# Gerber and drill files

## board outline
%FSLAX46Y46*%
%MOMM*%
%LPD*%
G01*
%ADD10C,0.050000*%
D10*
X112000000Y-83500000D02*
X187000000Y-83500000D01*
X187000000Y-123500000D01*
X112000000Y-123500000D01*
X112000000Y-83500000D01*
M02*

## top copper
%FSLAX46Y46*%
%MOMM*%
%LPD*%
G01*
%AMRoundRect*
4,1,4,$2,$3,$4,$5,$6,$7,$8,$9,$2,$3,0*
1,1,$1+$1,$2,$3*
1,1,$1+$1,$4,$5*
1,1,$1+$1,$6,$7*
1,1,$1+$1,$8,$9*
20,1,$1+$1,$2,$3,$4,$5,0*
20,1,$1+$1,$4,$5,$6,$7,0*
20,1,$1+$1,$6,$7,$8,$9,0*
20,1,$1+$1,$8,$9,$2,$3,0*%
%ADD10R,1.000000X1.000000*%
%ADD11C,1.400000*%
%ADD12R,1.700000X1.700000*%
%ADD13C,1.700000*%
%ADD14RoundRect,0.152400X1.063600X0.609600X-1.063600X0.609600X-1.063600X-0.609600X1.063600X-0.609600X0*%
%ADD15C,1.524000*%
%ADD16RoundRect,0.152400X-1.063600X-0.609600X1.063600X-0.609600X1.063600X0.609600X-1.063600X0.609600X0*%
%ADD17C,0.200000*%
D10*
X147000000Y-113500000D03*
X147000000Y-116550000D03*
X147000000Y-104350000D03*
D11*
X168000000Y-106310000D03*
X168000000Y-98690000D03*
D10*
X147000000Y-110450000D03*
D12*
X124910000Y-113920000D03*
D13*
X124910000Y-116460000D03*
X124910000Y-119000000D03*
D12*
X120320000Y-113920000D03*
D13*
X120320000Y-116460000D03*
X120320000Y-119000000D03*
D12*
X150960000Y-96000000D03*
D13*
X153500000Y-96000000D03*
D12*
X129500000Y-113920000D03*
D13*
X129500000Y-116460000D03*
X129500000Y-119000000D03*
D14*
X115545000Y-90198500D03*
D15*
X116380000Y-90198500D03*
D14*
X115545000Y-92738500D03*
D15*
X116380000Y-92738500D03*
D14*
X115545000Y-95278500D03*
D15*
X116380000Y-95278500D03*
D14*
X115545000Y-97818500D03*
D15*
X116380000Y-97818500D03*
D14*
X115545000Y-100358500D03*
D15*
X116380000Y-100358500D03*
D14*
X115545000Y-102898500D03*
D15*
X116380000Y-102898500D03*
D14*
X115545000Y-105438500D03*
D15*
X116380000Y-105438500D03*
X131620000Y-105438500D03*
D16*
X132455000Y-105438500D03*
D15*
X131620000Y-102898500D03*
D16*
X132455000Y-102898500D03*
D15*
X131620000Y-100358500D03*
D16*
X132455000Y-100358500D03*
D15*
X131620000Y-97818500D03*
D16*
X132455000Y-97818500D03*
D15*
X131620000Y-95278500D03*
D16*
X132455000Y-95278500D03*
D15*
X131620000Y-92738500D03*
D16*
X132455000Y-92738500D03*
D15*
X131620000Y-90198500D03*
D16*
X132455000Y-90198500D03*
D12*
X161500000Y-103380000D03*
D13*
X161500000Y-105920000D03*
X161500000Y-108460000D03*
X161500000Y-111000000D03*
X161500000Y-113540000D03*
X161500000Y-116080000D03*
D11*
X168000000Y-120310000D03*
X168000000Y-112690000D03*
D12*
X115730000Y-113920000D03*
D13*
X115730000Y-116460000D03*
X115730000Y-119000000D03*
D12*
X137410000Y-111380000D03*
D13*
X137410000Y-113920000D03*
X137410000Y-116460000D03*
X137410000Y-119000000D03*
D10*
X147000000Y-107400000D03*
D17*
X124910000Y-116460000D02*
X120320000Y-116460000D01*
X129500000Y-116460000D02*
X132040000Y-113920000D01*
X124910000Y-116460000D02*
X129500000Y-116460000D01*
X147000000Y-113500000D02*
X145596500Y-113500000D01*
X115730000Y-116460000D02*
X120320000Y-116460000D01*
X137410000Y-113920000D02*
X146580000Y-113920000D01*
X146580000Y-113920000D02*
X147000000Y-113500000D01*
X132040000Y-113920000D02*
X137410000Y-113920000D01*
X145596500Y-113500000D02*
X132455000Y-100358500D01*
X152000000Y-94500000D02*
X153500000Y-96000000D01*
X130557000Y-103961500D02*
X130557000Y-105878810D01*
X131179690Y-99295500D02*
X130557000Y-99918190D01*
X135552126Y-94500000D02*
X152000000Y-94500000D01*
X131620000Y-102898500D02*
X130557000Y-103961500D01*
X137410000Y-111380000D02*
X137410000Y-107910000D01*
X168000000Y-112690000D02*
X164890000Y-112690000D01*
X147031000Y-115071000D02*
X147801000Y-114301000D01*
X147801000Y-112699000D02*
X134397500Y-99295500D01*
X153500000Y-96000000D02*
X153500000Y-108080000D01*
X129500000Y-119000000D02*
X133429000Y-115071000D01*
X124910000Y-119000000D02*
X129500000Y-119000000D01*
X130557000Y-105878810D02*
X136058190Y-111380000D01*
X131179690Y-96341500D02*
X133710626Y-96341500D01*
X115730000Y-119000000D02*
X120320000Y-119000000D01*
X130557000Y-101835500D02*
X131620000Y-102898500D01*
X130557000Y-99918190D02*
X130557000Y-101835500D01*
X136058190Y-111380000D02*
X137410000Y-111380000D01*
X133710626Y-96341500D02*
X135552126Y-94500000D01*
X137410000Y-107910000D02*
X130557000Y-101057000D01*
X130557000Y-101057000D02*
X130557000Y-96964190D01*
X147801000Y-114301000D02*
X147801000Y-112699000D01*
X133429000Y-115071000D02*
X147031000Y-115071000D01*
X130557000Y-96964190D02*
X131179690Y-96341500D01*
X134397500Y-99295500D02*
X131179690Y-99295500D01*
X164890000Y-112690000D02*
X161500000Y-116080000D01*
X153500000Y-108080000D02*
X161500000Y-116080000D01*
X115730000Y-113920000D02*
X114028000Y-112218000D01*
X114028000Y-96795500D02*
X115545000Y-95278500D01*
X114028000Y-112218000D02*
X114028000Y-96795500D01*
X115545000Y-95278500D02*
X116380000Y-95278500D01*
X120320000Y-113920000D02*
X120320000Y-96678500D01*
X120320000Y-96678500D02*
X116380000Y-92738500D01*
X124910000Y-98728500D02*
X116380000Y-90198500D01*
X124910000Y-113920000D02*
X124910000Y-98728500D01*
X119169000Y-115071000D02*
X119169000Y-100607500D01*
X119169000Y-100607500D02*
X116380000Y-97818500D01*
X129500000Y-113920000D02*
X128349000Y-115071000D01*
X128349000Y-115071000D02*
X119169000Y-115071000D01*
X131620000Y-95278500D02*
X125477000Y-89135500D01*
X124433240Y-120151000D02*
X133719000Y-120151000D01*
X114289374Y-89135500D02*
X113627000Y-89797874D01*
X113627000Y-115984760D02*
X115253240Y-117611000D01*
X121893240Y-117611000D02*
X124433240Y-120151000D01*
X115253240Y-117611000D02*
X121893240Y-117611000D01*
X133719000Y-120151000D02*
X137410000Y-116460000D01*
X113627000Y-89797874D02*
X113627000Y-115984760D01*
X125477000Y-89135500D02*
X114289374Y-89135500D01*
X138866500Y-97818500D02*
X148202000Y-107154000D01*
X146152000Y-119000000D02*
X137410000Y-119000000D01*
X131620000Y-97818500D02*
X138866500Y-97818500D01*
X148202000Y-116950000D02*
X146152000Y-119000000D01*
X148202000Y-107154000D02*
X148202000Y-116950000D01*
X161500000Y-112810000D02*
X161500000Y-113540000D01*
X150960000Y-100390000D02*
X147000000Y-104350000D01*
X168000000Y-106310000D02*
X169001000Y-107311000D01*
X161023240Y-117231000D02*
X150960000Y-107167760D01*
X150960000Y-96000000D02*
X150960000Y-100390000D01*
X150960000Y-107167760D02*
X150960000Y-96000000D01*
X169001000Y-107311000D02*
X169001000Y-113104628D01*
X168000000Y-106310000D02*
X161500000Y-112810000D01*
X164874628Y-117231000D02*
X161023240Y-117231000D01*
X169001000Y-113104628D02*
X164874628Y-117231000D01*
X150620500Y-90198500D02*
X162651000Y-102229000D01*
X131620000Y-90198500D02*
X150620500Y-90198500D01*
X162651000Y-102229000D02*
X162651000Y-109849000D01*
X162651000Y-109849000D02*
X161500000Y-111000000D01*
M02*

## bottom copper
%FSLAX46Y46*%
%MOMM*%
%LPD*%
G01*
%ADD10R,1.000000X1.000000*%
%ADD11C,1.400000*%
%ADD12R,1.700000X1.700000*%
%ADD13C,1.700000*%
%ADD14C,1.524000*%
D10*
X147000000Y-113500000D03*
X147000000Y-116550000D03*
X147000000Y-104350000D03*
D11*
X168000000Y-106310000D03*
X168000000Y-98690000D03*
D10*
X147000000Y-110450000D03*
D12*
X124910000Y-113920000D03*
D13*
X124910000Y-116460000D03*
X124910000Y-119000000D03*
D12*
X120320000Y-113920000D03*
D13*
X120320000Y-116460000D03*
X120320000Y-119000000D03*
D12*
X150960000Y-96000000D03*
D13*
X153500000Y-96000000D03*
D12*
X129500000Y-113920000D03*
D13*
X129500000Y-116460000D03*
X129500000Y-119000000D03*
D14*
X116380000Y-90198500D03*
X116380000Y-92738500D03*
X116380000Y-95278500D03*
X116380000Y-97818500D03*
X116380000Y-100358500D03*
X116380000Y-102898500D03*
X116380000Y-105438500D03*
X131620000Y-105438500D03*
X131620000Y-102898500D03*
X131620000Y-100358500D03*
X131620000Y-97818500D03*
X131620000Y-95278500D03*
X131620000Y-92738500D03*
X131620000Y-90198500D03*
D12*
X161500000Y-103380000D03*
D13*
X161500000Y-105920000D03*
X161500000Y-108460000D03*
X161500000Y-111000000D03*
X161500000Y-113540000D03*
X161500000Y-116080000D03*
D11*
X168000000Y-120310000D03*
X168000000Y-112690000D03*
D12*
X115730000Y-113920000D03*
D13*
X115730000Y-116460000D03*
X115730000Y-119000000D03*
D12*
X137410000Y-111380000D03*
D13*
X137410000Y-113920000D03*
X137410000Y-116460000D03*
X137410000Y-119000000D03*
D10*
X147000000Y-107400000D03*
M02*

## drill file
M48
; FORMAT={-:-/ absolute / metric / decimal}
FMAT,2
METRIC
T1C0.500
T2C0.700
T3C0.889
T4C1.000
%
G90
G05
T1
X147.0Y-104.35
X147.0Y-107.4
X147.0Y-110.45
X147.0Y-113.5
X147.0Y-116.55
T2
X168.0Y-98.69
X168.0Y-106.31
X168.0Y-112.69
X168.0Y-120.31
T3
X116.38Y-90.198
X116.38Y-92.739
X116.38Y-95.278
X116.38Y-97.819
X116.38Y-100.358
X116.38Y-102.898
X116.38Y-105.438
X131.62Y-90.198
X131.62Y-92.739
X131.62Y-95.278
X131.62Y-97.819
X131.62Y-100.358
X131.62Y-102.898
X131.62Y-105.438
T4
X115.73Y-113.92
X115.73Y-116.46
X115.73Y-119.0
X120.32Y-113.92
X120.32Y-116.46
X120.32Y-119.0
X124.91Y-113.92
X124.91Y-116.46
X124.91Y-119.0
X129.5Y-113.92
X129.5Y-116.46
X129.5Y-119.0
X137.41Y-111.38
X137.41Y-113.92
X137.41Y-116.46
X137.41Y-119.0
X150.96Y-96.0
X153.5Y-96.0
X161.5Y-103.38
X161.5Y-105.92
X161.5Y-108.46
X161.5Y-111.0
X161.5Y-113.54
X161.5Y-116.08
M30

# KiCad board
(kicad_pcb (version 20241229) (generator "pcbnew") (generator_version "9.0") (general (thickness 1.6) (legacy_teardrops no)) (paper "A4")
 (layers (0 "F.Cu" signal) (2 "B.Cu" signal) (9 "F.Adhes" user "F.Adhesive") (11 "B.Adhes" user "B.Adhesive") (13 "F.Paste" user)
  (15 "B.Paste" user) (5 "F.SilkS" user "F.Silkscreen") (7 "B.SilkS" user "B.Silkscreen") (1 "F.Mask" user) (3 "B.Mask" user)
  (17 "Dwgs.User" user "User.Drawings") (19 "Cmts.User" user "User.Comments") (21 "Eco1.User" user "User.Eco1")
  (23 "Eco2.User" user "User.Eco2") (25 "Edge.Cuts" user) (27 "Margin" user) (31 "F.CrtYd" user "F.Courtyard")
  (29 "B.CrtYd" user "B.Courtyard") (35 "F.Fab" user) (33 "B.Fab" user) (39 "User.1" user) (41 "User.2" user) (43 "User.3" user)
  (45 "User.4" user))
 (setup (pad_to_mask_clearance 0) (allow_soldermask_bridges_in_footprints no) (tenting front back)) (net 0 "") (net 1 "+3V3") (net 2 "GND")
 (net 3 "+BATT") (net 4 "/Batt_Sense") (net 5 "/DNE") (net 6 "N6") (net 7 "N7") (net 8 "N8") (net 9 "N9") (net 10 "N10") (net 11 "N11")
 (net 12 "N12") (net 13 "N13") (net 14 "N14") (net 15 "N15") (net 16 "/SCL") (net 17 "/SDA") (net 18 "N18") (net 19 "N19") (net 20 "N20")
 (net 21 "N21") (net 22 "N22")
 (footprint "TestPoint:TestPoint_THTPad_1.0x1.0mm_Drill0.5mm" (layer "F.Cu") (at 147 113.5)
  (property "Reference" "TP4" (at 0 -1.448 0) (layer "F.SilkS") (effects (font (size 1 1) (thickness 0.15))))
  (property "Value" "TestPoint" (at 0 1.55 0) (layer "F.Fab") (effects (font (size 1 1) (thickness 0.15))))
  (pad "1" thru_hole rect (at 0 0) (size 1 1) (drill 0.5) (layers "*.Cu" "*.Mask") (remove_unused_layers no) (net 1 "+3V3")))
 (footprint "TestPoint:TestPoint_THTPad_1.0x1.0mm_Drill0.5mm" (layer "F.Cu") (at 147 116.55)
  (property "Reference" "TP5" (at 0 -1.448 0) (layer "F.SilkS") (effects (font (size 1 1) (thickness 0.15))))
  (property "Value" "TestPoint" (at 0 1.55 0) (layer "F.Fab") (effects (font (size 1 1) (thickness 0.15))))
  (pad "1" thru_hole rect (at 0 0) (size 1 1) (drill 0.5) (layers "*.Cu" "*.Mask") (remove_unused_layers no) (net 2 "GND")))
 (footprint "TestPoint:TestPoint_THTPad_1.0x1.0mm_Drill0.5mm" (layer "F.Cu") (at 147 104.35)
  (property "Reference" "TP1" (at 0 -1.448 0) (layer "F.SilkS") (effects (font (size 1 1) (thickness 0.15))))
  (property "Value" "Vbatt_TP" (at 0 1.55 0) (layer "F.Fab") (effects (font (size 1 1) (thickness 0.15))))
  (pad "1" thru_hole rect (at 0 0) (size 1 1) (drill 0.5) (layers "*.Cu" "*.Mask") (remove_unused_layers no) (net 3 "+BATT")))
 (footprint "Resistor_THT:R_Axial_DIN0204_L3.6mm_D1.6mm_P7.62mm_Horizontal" (layer "F.Cu") (at 168 106.31 90)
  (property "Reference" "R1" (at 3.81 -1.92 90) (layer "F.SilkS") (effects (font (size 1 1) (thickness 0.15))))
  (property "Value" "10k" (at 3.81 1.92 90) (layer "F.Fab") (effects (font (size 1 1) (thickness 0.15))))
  (pad "1" thru_hole circle (at 0 0 90) (size 1.4 1.4) (drill 0.7) (layers "*.Cu" "*.Mask") (remove_unused_layers no) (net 3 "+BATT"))
  (pad "2" thru_hole circle (at 7.62 0 90) (size 1.4 1.4) (drill 0.7) (layers "*.Cu" "*.Mask") (remove_unused_layers no)
   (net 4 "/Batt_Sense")))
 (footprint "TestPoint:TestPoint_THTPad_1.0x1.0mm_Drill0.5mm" (layer "F.Cu") (at 147 110.45)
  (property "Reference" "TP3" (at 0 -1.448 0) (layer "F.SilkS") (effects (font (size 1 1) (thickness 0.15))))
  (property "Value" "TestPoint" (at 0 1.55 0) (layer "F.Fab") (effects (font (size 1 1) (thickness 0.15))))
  (pad "1" thru_hole rect (at 0 0) (size 1 1) (drill 0.5) (layers "*.Cu" "*.Mask") (remove_unused_layers no) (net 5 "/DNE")))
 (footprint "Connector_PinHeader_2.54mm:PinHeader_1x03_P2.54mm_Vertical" (layer "F.Cu") (at 124.91 113.92)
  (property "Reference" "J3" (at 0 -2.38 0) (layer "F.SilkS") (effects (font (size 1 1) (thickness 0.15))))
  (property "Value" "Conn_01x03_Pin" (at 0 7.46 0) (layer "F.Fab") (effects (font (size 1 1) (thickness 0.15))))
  (pad "1" thru_hole rect (at 0 0) (size 1.7 1.7) (drill 1) (layers "*.Cu" "*.Mask") (remove_unused_layers no) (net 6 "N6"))
  (pad "2" thru_hole circle (at 0 2.54) (size 1.7 1.7) (drill 1) (layers "*.Cu" "*.Mask") (remove_unused_layers no) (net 1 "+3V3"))
  (pad "3" thru_hole circle (at 0 5.08) (size 1.7 1.7) (drill 1) (layers "*.Cu" "*.Mask") (remove_unused_layers no) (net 2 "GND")))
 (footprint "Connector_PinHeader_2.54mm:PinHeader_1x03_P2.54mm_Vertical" (layer "F.Cu") (at 120.32 113.92)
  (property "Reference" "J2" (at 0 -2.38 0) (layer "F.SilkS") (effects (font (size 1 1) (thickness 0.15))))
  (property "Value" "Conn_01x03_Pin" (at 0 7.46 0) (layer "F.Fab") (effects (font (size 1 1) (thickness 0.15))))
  (pad "1" thru_hole rect (at 0 0) (size 1.7 1.7) (drill 1) (layers "*.Cu" "*.Mask") (remove_unused_layers no) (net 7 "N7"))
  (pad "2" thru_hole circle (at 0 2.54) (size 1.7 1.7) (drill 1) (layers "*.Cu" "*.Mask") (remove_unused_layers no) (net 1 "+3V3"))
  (pad "3" thru_hole circle (at 0 5.08) (size 1.7 1.7) (drill 1) (layers "*.Cu" "*.Mask") (remove_unused_layers no) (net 2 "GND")))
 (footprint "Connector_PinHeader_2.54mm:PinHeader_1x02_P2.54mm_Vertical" (layer "F.Cu") (at 150.96 96 90)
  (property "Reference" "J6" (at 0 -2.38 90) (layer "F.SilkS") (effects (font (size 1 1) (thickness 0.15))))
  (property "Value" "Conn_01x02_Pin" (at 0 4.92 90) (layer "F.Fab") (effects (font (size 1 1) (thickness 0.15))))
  (pad "1" thru_hole rect (at 0 0 90) (size 1.7 1.7) (drill 1) (layers "*.Cu" "*.Mask") (remove_unused_layers no) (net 3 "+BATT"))
  (pad "2" thru_hole circle (at 0 2.54 90) (size 1.7 1.7) (drill 1) (layers "*.Cu" "*.Mask") (remove_unused_layers no) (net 2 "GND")))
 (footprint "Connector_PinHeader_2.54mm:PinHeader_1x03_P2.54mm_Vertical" (layer "F.Cu") (at 129.5 113.92)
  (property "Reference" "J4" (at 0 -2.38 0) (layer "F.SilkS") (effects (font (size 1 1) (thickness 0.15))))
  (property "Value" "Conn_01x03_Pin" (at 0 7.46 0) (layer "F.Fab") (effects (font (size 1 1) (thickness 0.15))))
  (pad "1" thru_hole rect (at 0 0) (size 1.7 1.7) (drill 1) (layers "*.Cu" "*.Mask") (remove_unused_layers no) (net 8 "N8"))
  (pad "2" thru_hole circle (at 0 2.54) (size 1.7 1.7) (drill 1) (layers "*.Cu" "*.Mask") (remove_unused_layers no) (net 1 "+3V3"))
  (pad "3" thru_hole circle (at 0 5.08) (size 1.7 1.7) (drill 1) (layers "*.Cu" "*.Mask") (remove_unused_layers no) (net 2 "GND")))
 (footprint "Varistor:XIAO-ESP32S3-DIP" (layer "F.Cu") (at 124 97.8185)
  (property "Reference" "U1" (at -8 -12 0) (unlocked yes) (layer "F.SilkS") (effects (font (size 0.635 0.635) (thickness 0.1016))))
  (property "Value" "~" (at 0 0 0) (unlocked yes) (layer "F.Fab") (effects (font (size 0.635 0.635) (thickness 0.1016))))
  (pad "1" smd roundrect (at -8.455 -7.62 180) (size 2.432 1.524) (layers "F.Cu" "F.Mask") (roundrect_rratio 0.1) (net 6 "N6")
   (thermal_bridge_angle 45))
  (pad "1" thru_hole circle (at -7.62 -7.62 180) (size 1.524 1.524) (drill 0.889) (layers "*.Cu" "*.Mask") (remove_unused_layers no)
   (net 6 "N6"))
  (pad "2" smd roundrect (at -8.455 -5.08 180) (size 2.432 1.524) (layers "F.Cu" "F.Mask") (roundrect_rratio 0.1) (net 7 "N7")
   (thermal_bridge_angle 45))
  (pad "2" thru_hole circle (at -7.62 -5.08 180) (size 1.524 1.524) (drill 0.889) (layers "*.Cu" "*.Mask") (remove_unused_layers no)
   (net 7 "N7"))
  (pad "3" smd roundrect (at -8.455 -2.54 180) (size 2.432 1.524) (layers "F.Cu" "F.Mask") (roundrect_rratio 0.1) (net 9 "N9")
   (thermal_bridge_angle 45))
  (pad "3" thru_hole circle (at -7.62 -2.54 180) (size 1.524 1.524) (drill 0.889) (layers "*.Cu" "*.Mask") (remove_unused_layers no)
   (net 9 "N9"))
  (pad "4" smd roundrect (at -8.455 0 180) (size 2.432 1.524) (layers "F.Cu" "F.Mask") (roundrect_rratio 0.1) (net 8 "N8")
   (thermal_bridge_angle 45))
  (pad "4" thru_hole circle (at -7.62 0 180) (size 1.524 1.524) (drill 0.889) (layers "*.Cu" "*.Mask") (remove_unused_layers no)
   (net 8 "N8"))
  (pad "5" smd roundrect (at -8.455 2.54 180) (size 2.432 1.524) (layers "F.Cu" "F.Mask") (roundrect_rratio 0.1) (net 4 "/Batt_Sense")
   (thermal_bridge_angle 45))
  (pad "5" thru_hole circle (at -7.62 2.54 180) (size 1.524 1.524) (drill 0.889) (layers "*.Cu" "*.Mask") (remove_unused_layers no)
   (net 4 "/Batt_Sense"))
  (pad "6" smd roundrect (at -8.455 5.08 180) (size 2.432 1.524) (layers "F.Cu" "F.Mask") (roundrect_rratio 0.1) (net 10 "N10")
   (thermal_bridge_angle 45))
  (pad "6" thru_hole circle (at -7.62 5.08 180) (size 1.524 1.524) (drill 0.889) (layers "*.Cu" "*.Mask") (remove_unused_layers no)
   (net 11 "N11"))
  (pad "7" smd roundrect (at -8.455 7.62 180) (size 2.432 1.524) (layers "F.Cu" "F.Mask") (roundrect_rratio 0.1) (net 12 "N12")
   (thermal_bridge_angle 45))
  (pad "7" thru_hole circle (at -7.62 7.62 180) (size 1.524 1.524) (drill 0.889) (layers "*.Cu" "*.Mask") (remove_unused_layers no)
   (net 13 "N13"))
  (pad "8" thru_hole circle (at 7.62 7.62) (size 1.524 1.524) (drill 0.889) (layers "*.Cu" "*.Mask") (remove_unused_layers no)
   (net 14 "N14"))
  (pad "8" smd roundrect (at 8.455 7.62) (size 2.432 1.524) (layers "F.Cu" "F.Mask") (roundrect_rratio 0.1) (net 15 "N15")
   (thermal_bridge_angle 45))
  (pad "9" thru_hole circle (at 7.62 5.08) (size 1.524 1.524) (drill 0.889) (layers "*.Cu" "*.Mask") (remove_unused_layers no) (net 2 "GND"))
  (pad "9" smd roundrect (at 8.455 5.08) (size 2.432 1.524) (layers "F.Cu" "F.Mask") (roundrect_rratio 0.1) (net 2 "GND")
   (thermal_bridge_angle 45))
  (pad "10" thru_hole circle (at 7.62 2.54) (size 1.524 1.524) (drill 0.889) (layers "*.Cu" "*.Mask") (remove_unused_layers no)
   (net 1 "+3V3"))
  (pad "10" smd roundrect (at 8.455 2.54) (size 2.432 1.524) (layers "F.Cu" "F.Mask") (roundrect_rratio 0.1) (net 1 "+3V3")
   (thermal_bridge_angle 45))
  (pad "11" thru_hole circle (at 7.62 0) (size 1.524 1.524) (drill 0.889) (layers "*.Cu" "*.Mask") (remove_unused_layers no) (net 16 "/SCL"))
  (pad "11" smd roundrect (at 8.455 0) (size 2.432 1.524) (layers "F.Cu" "F.Mask") (roundrect_rratio 0.1) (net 16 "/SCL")
   (thermal_bridge_angle 45))
  (pad "12" thru_hole circle (at 7.62 -2.54) (size 1.524 1.524) (drill 0.889) (layers "*.Cu" "*.Mask") (remove_unused_layers no)
   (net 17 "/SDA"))
  (pad "12" smd roundrect (at 8.455 -2.54) (size 2.432 1.524) (layers "F.Cu" "F.Mask") (roundrect_rratio 0.1) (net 17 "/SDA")
   (thermal_bridge_angle 45))
  (pad "13" thru_hole circle (at 7.62 -5.08) (size 1.524 1.524) (drill 0.889) (layers "*.Cu" "*.Mask") (remove_unused_layers no)
   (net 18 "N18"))
  (pad "13" smd roundrect (at 8.455 -5.08) (size 2.432 1.524) (layers "F.Cu" "F.Mask") (roundrect_rratio 0.1) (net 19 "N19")
   (thermal_bridge_angle 45))
  (pad "14" thru_hole circle (at 7.62 -7.62) (size 1.524 1.524) (drill 0.889) (layers "*.Cu" "*.Mask") (remove_unused_layers no)
   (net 5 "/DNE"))
  (pad "14" smd roundrect (at 8.455 -7.62) (size 2.432 1.524) (layers "F.Cu" "F.Mask") (roundrect_rratio 0.1) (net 5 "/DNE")
   (thermal_bridge_angle 45)))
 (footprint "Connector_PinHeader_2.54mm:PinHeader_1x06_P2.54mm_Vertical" (layer "F.Cu") (at 161.5 103.38)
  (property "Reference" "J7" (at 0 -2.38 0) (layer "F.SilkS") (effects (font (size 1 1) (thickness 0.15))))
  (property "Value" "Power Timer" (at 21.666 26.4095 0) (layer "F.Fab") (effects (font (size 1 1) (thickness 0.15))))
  (pad "1" thru_hole rect (at 0 0) (size 1.7 1.7) (drill 1) (layers "*.Cu" "*.Mask") (remove_unused_layers no) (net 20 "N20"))
  (pad "2" thru_hole circle (at 0 2.54) (size 1.7 1.7) (drill 1) (layers "*.Cu" "*.Mask") (remove_unused_layers no) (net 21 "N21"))
  (pad "3" thru_hole circle (at 0 5.08) (size 1.7 1.7) (drill 1) (layers "*.Cu" "*.Mask") (remove_unused_layers no) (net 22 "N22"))
  (pad "4" thru_hole circle (at 0 7.62) (size 1.7 1.7) (drill 1) (layers "*.Cu" "*.Mask") (remove_unused_layers no) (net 5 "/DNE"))
  (pad "5" thru_hole circle (at 0 10.16) (size 1.7 1.7) (drill 1) (layers "*.Cu" "*.Mask") (remove_unused_layers no) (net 3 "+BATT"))
  (pad "6" thru_hole circle (at 0 12.7) (size 1.7 1.7) (drill 1) (layers "*.Cu" "*.Mask") (remove_unused_layers no) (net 2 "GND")))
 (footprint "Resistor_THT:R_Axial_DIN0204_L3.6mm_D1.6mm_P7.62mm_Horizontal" (layer "F.Cu") (at 168 120.31 90)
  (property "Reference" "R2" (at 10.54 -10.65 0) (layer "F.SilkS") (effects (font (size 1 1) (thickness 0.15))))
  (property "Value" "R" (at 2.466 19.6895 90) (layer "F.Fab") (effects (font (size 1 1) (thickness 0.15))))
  (pad "1" thru_hole circle (at 0 0 90) (size 1.4 1.4) (drill 0.7) (layers "*.Cu" "*.Mask") (remove_unused_layers no) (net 4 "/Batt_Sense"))
  (pad "2" thru_hole circle (at 7.62 0 90) (size 1.4 1.4) (drill 0.7) (layers "*.Cu" "*.Mask") (remove_unused_layers no) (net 2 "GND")))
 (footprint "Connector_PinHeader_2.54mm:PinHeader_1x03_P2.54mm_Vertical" (layer "F.Cu") (at 115.73 113.92)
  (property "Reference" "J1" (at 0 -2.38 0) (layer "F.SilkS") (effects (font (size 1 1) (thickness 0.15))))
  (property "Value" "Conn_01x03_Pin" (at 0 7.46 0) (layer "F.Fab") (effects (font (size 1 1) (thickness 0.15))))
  (pad "1" thru_hole rect (at 0 0) (size 1.7 1.7) (drill 1) (layers "*.Cu" "*.Mask") (remove_unused_layers no) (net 9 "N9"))
  (pad "2" thru_hole circle (at 0 2.54) (size 1.7 1.7) (drill 1) (layers "*.Cu" "*.Mask") (remove_unused_layers no) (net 1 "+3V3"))
  (pad "3" thru_hole circle (at 0 5.08) (size 1.7 1.7) (drill 1) (layers "*.Cu" "*.Mask") (remove_unused_layers no) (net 2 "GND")))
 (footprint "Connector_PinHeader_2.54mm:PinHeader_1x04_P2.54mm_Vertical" (layer "F.Cu") (at 137.41 111.38)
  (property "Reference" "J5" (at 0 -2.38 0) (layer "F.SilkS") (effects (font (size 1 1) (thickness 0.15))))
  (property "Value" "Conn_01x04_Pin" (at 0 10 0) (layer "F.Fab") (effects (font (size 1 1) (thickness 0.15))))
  (pad "1" thru_hole rect (at 0 0) (size 1.7 1.7) (drill 1) (layers "*.Cu" "*.Mask") (remove_unused_layers no) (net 2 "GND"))
  (pad "2" thru_hole circle (at 0 2.54) (size 1.7 1.7) (drill 1) (layers "*.Cu" "*.Mask") (remove_unused_layers no) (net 1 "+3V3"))
  (pad "3" thru_hole circle (at 0 5.08) (size 1.7 1.7) (drill 1) (layers "*.Cu" "*.Mask") (remove_unused_layers no) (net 17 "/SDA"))
  (pad "4" thru_hole circle (at 0 7.62) (size 1.7 1.7) (drill 1) (layers "*.Cu" "*.Mask") (remove_unused_layers no) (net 16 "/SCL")))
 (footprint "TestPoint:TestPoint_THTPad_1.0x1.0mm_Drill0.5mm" (layer "F.Cu") (at 147 107.4)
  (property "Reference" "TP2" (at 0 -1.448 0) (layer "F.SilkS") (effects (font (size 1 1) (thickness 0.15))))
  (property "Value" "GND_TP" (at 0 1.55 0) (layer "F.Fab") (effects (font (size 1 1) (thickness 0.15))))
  (pad "1" thru_hole rect (at 0 0) (size 1 1) (drill 0.5) (layers "*.Cu" "*.Mask") (remove_unused_layers no) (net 2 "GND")))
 (gr_rect (start 112 83.5) (end 187 123.5) (stroke (width 0.05) (type default)) (fill no) (layer "Edge.Cuts"))
 (segment (start 124.91 116.46) (end 120.32 116.46) (width 0.2) (layer "F.Cu") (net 1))
 (segment (start 129.5 116.46) (end 132.04 113.92) (width 0.2) (layer "F.Cu") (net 1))
 (segment (start 124.91 116.46) (end 129.5 116.46) (width 0.2) (layer "F.Cu") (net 1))
 (segment (start 147 113.5) (end 145.5965 113.5) (width 0.2) (layer "F.Cu") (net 1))
 (segment (start 115.73 116.46) (end 120.32 116.46) (width 0.2) (layer "F.Cu") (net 1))
 (segment (start 137.41 113.92) (end 146.58 113.92) (width 0.2) (layer "F.Cu") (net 1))
 (segment (start 146.58 113.92) (end 147 113.5) (width 0.2) (layer "F.Cu") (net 1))
 (segment (start 132.04 113.92) (end 137.41 113.92) (width 0.2) (layer "F.Cu") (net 1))
 (segment (start 145.5965 113.5) (end 132.455 100.3585) (width 0.2) (layer "F.Cu") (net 1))
 (segment (start 152 94.5) (end 153.5 96) (width 0.2) (layer "F.Cu") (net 2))
 (segment (start 130.557 103.9615) (end 130.557 105.87881) (width 0.2) (layer "F.Cu") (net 2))
 (segment (start 131.17969 99.2955) (end 130.557 99.91819) (width 0.2) (layer "F.Cu") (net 2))
 (segment (start 135.552126 94.5) (end 152 94.5) (width 0.2) (layer "F.Cu") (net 2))
 (segment (start 131.62 102.8985) (end 130.557 103.9615) (width 0.2) (layer "F.Cu") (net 2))
 (segment (start 137.41 111.38) (end 137.41 107.91) (width 0.2) (layer "F.Cu") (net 2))
 (segment (start 168 112.69) (end 164.89 112.69) (width 0.2) (layer "F.Cu") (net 2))
 (segment (start 147.031 115.071) (end 147.801 114.301) (width 0.2) (layer "F.Cu") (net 2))
 (segment (start 147.801 112.699) (end 134.3975 99.2955) (width 0.2) (layer "F.Cu") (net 2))
 (segment (start 153.5 96) (end 153.5 108.08) (width 0.2) (layer "F.Cu") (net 2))
 (segment (start 129.5 119) (end 133.429 115.071) (width 0.2) (layer "F.Cu") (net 2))
 (segment (start 124.91 119) (end 129.5 119) (width 0.2) (layer "F.Cu") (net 2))
 (segment (start 130.557 105.87881) (end 136.05819 111.38) (width 0.2) (layer "F.Cu") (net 2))
 (segment (start 131.17969 96.3415) (end 133.710626 96.3415) (width 0.2) (layer "F.Cu") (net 2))
 (segment (start 115.73 119) (end 120.32 119) (width 0.2) (layer "F.Cu") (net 2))
 (segment (start 130.557 101.8355) (end 131.62 102.8985) (width 0.2) (layer "F.Cu") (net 2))
 (segment (start 130.557 99.91819) (end 130.557 101.8355) (width 0.2) (layer "F.Cu") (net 2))
 (segment (start 136.05819 111.38) (end 137.41 111.38) (width 0.2) (layer "F.Cu") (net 2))
 (segment (start 133.710626 96.3415) (end 135.552126 94.5) (width 0.2) (layer "F.Cu") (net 2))
 (segment (start 137.41 107.91) (end 130.557 101.057) (width 0.2) (layer "F.Cu") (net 2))
 (segment (start 130.557 101.057) (end 130.557 96.96419) (width 0.2) (layer "F.Cu") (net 2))
 (segment (start 147.801 114.301) (end 147.801 112.699) (width 0.2) (layer "F.Cu") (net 2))
 (segment (start 133.429 115.071) (end 147.031 115.071) (width 0.2) (layer "F.Cu") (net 2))
 (segment (start 130.557 96.96419) (end 131.17969 96.3415) (width 0.2) (layer "F.Cu") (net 2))
 (segment (start 134.3975 99.2955) (end 131.17969 99.2955) (width 0.2) (layer "F.Cu") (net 2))
 (segment (start 164.89 112.69) (end 161.5 116.08) (width 0.2) (layer "F.Cu") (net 2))
 (segment (start 153.5 108.08) (end 161.5 116.08) (width 0.2) (layer "F.Cu") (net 2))
 (segment (start 115.73 113.92) (end 114.028 112.218) (width 0.2) (layer "F.Cu") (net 9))
 (segment (start 114.028 96.7955) (end 115.545 95.2785) (width 0.2) (layer "F.Cu") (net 9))
 (segment (start 114.028 112.218) (end 114.028 96.7955) (width 0.2) (layer "F.Cu") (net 9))
 (segment (start 115.545 95.2785) (end 116.38 95.2785) (width 0.2) (layer "F.Cu") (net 9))
 (segment (start 120.32 113.92) (end 120.32 96.6785) (width 0.2) (layer "F.Cu") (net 7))
 (segment (start 120.32 96.6785) (end 116.38 92.7385) (width 0.2) (layer "F.Cu") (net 7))
 (segment (start 124.91 98.7285) (end 116.38 90.1985) (width 0.2) (layer "F.Cu") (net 6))
 (segment (start 124.91 113.92) (end 124.91 98.7285) (width 0.2) (layer "F.Cu") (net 6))
 (segment (start 119.169 115.071) (end 119.169 100.6075) (width 0.2) (layer "F.Cu") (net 8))
 (segment (start 119.169 100.6075) (end 116.38 97.8185) (width 0.2) (layer "F.Cu") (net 8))
 (segment (start 129.5 113.92) (end 128.349 115.071) (width 0.2) (layer "F.Cu") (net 8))
 (segment (start 128.349 115.071) (end 119.169 115.071) (width 0.2) (layer "F.Cu") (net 8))
 (segment (start 131.62 95.2785) (end 125.477 89.1355) (width 0.2) (layer "F.Cu") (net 17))
 (segment (start 124.43324 120.151) (end 133.719 120.151) (width 0.2) (layer "F.Cu") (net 17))
 (segment (start 114.289374 89.1355) (end 113.627 89.797874) (width 0.2) (layer "F.Cu") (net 17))
 (segment (start 113.627 115.98476) (end 115.25324 117.611) (width 0.2) (layer "F.Cu") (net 17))
 (segment (start 121.89324 117.611) (end 124.43324 120.151) (width 0.2) (layer "F.Cu") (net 17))
 (segment (start 115.25324 117.611) (end 121.89324 117.611) (width 0.2) (layer "F.Cu") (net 17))
 (segment (start 133.719 120.151) (end 137.41 116.46) (width 0.2) (layer "F.Cu") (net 17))
 (segment (start 113.627 89.797874) (end 113.627 115.98476) (width 0.2) (layer "F.Cu") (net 17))
 (segment (start 125.477 89.1355) (end 114.289374 89.1355) (width 0.2) (layer "F.Cu") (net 17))
 (segment (start 138.8665 97.8185) (end 148.202 107.154) (width 0.2) (layer "F.Cu") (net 16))
 (segment (start 146.152 119) (end 137.41 119) (width 0.2) (layer "F.Cu") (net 16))
 (segment (start 131.62 97.8185) (end 138.8665 97.8185) (width 0.2) (layer "F.Cu") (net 16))
 (segment (start 148.202 116.95) (end 146.152 119) (width 0.2) (layer "F.Cu") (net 16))
 (segment (start 148.202 107.154) (end 148.202 116.95) (width 0.2) (layer "F.Cu") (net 16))
 (segment (start 161.5 112.81) (end 161.5 113.54) (width 0.2) (layer "F.Cu") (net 3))
 (segment (start 150.96 100.39) (end 147 104.35) (width 0.2) (layer "F.Cu") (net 3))
 (segment (start 168 106.31) (end 169.001 107.311) (width 0.2) (layer "F.Cu") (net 3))
 (segment (start 161.02324 117.231) (end 150.96 107.16776) (width 0.2) (layer "F.Cu") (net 3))
 (segment (start 150.96 96) (end 150.96 100.39) (width 0.2) (layer "F.Cu") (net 3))
 (segment (start 150.96 107.16776) (end 150.96 96) (width 0.2) (layer "F.Cu") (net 3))
 (segment (start 169.001 107.311) (end 169.001 113.104628) (width 0.2) (layer "F.Cu") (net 3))
 (segment (start 168 106.31) (end 161.5 112.81) (width 0.2) (layer "F.Cu") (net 3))
 (segment (start 164.874628 117.231) (end 161.02324 117.231) (width 0.2) (layer "F.Cu") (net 3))
 (segment (start 169.001 113.104628) (end 164.874628 117.231) (width 0.2) (layer "F.Cu") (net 3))
 (segment (start 150.6205 90.1985) (end 162.651 102.229) (width 0.2) (layer "F.Cu") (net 5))
 (segment (start 131.62 90.1985) (end 150.6205 90.1985) (width 0.2) (layer "F.Cu") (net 5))
 (segment (start 162.651 102.229) (end 162.651 109.849) (width 0.2) (layer "F.Cu") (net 5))
 (segment (start 162.651 109.849) (end 161.5 111) (width 0.2) (layer "F.Cu") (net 5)))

